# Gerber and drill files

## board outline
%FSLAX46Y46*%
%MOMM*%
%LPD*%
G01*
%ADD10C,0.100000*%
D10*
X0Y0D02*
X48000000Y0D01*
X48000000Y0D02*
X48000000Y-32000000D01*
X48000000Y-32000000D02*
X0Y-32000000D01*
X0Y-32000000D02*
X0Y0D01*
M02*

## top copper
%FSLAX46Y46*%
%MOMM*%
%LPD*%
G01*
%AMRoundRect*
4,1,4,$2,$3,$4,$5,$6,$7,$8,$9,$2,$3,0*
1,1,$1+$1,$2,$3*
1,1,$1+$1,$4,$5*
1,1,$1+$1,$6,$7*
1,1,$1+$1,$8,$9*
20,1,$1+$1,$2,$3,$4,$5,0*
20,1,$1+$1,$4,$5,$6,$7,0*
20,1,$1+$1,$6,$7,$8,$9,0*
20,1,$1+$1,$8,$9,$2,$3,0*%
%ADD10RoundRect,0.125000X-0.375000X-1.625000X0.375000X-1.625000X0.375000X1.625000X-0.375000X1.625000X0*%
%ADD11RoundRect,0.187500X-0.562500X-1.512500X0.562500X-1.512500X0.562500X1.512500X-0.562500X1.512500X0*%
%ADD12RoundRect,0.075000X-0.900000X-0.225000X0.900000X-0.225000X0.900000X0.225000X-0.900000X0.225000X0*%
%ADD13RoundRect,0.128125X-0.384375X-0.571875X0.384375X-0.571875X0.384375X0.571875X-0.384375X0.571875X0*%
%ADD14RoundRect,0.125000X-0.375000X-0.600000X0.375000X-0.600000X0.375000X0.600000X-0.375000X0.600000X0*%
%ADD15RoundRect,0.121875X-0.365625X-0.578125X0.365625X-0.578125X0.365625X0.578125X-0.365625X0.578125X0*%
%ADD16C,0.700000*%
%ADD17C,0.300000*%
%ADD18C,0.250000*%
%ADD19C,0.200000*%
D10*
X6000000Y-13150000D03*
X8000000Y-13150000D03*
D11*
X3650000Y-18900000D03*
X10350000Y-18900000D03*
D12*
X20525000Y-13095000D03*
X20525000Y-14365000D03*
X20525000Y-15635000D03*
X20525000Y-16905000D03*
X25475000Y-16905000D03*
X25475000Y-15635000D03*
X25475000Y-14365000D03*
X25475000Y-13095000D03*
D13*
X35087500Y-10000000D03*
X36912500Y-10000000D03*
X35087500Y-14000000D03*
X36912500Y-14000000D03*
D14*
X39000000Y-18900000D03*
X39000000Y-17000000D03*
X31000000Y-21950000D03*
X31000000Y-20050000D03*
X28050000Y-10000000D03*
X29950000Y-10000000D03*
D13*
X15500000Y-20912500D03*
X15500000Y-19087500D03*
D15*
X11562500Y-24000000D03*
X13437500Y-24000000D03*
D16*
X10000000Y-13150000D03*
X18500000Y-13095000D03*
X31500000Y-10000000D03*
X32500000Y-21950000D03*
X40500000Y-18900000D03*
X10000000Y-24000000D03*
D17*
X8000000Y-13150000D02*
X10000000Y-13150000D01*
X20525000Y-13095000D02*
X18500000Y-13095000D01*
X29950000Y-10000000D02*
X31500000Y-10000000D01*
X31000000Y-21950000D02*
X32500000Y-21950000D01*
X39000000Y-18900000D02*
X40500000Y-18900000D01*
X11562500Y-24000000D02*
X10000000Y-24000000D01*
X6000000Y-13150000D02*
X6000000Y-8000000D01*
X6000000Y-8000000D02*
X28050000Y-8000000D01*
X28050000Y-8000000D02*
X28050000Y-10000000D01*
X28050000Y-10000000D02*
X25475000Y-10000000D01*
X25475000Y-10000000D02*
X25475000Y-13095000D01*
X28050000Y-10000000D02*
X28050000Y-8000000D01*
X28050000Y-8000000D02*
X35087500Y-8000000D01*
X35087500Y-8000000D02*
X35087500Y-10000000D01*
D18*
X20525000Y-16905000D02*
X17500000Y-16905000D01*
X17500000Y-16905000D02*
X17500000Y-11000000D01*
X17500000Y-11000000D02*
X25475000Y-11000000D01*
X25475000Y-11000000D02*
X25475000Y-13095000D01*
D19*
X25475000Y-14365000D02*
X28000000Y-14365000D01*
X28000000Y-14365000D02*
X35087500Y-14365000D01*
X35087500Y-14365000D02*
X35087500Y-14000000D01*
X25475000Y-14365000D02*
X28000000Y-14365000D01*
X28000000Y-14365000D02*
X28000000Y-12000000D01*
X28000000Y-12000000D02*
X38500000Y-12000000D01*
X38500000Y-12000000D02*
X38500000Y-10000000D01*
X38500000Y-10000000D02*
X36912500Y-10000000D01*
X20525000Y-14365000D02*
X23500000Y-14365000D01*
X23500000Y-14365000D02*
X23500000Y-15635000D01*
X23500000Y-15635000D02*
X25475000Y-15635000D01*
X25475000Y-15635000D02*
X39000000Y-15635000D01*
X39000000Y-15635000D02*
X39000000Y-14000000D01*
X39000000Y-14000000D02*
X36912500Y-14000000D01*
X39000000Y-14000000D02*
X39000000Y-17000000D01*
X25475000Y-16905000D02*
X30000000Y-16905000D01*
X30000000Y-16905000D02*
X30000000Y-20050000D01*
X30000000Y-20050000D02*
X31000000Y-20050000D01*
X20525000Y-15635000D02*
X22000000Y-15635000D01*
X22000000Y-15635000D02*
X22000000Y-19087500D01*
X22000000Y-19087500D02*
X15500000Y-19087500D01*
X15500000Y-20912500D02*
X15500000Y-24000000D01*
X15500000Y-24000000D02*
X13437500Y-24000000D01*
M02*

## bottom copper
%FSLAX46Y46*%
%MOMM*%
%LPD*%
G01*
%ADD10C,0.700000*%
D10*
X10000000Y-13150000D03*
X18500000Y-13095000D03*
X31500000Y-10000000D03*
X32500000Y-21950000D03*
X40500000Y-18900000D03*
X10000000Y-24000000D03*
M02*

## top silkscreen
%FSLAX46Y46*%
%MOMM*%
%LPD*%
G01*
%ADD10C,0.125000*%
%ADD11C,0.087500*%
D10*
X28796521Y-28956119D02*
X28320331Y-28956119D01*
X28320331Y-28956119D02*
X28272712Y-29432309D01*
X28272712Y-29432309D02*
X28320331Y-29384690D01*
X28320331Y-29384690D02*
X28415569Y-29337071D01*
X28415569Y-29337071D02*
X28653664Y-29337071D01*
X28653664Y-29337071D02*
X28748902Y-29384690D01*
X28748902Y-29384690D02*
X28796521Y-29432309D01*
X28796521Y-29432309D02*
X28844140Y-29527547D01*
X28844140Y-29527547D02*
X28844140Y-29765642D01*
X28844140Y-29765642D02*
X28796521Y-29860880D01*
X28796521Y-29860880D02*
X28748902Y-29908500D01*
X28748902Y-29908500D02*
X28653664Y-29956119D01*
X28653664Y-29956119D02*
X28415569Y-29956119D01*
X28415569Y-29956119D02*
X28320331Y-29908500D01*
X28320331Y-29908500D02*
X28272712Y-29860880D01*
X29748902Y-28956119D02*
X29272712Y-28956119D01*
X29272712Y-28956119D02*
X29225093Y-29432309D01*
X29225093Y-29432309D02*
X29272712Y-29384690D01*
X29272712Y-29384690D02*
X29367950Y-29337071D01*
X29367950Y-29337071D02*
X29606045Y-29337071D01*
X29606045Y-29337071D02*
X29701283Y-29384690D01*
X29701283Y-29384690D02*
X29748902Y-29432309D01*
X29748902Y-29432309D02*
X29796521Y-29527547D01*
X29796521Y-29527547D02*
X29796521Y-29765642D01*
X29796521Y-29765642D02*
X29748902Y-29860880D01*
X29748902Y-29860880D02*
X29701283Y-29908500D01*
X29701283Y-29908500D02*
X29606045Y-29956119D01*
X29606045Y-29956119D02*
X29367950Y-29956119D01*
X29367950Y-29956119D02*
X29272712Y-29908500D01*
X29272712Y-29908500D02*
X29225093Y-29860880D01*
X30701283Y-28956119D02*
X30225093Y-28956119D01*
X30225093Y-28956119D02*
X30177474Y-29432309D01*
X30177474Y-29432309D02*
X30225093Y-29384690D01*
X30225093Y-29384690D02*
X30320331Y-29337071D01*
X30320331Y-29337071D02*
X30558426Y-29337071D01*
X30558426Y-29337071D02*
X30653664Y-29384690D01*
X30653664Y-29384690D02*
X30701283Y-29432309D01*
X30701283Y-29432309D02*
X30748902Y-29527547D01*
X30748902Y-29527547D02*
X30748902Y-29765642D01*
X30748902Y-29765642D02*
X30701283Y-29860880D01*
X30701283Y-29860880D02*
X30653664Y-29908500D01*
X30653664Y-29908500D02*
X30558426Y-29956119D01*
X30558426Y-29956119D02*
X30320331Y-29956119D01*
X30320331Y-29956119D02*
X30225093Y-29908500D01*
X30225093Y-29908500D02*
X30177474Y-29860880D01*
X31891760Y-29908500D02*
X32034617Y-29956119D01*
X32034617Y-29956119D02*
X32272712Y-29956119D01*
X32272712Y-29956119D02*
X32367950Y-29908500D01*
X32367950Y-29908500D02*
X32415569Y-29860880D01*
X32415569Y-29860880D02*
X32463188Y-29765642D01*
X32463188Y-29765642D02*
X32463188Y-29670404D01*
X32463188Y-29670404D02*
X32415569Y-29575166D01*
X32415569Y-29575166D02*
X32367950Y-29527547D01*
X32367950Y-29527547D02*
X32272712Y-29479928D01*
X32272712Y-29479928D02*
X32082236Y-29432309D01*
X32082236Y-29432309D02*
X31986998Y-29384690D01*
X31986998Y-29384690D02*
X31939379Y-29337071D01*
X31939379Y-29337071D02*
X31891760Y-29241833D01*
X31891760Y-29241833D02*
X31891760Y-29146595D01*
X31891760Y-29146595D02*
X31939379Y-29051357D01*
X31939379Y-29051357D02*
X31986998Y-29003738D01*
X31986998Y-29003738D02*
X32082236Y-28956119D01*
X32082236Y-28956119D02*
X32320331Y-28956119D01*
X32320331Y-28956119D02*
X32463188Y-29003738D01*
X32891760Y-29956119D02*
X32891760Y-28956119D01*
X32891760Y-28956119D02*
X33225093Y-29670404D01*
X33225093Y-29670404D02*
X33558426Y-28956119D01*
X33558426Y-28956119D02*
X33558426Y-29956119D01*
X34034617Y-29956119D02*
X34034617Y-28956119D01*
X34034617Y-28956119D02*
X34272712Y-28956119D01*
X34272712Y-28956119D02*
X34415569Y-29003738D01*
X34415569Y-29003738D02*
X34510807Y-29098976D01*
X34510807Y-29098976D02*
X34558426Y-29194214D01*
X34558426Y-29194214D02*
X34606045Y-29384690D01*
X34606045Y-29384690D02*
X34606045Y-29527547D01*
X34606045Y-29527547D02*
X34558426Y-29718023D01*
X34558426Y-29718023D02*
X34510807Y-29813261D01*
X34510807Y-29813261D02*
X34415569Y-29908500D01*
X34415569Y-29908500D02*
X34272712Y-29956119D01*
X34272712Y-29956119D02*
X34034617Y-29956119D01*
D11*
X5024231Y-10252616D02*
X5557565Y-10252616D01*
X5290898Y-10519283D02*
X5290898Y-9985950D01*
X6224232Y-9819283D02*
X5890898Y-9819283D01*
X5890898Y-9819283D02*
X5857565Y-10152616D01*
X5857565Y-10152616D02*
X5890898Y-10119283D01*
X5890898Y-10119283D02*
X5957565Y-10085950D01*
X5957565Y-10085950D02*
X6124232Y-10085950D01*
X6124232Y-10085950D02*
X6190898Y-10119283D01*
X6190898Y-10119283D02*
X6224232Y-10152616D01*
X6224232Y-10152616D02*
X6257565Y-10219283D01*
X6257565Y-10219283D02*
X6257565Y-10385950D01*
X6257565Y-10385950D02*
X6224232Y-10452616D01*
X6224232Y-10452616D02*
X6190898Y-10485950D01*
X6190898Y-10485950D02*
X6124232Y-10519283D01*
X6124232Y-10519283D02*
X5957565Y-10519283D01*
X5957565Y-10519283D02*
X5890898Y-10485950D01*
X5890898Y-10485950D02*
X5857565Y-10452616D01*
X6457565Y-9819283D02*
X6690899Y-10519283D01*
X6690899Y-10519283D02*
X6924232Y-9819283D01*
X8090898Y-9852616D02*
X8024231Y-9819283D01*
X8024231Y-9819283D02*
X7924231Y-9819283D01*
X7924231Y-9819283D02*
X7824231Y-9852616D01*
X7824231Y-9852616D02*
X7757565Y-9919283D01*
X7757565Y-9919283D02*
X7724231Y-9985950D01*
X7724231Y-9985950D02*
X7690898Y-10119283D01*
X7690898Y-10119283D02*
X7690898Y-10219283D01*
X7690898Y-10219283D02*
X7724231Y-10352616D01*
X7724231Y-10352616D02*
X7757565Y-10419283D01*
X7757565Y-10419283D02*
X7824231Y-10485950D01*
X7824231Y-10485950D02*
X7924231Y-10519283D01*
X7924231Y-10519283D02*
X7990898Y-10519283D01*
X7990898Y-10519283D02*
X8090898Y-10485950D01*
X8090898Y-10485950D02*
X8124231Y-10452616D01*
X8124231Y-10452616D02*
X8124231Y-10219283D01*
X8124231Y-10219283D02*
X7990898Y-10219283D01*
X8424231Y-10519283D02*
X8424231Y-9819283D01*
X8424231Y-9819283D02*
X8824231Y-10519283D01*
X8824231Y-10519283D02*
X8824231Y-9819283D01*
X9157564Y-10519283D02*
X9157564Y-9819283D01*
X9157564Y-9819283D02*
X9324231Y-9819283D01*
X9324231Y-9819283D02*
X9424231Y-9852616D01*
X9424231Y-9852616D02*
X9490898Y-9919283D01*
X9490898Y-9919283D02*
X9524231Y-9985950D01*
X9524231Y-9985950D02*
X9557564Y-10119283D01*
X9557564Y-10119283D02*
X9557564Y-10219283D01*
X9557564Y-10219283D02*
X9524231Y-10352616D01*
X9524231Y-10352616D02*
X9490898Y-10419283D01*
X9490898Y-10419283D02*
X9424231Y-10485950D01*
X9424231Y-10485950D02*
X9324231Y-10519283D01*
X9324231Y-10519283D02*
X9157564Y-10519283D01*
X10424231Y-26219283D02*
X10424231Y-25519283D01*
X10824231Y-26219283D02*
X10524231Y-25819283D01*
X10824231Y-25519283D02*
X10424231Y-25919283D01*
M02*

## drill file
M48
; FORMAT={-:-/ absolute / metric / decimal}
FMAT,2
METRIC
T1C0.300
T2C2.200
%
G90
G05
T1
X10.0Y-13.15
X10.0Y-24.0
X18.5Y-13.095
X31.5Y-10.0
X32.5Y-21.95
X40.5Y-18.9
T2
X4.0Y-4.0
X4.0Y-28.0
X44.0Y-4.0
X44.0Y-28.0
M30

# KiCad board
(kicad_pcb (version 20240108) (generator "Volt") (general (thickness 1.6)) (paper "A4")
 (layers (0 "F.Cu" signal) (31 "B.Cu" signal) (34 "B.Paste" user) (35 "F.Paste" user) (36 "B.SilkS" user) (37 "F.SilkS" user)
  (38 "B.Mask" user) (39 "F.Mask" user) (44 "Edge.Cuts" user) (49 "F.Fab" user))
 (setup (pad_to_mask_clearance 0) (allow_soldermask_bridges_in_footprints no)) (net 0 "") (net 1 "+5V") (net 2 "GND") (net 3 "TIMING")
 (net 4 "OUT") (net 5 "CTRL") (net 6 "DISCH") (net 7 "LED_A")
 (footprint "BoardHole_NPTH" (layer "F.Cu") (at 4 4)
  (pad "" np_thru_hole circle (at 0 0) (size 2.2 2.2) (drill 2.2) (layers "*.Cu" "*.Mask")))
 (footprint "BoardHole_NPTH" (layer "F.Cu") (at 44 4)
  (pad "" np_thru_hole circle (at 0 0) (size 2.2 2.2) (drill 2.2) (layers "*.Cu" "*.Mask")))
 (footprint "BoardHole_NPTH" (layer "F.Cu") (at 4 28)
  (pad "" np_thru_hole circle (at 0 0) (size 2.2 2.2) (drill 2.2) (layers "*.Cu" "*.Mask")))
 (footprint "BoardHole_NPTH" (layer "F.Cu") (at 44 28)
  (pad "" np_thru_hole circle (at 0 0) (size 2.2 2.2) (drill 2.2) (layers "*.Cu" "*.Mask")))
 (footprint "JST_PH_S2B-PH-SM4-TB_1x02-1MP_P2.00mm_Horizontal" (layer "F.Cu") (at 7 16)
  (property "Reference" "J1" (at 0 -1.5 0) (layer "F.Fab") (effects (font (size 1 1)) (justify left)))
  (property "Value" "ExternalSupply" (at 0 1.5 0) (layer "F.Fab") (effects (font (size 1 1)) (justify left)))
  (pad "1" smd roundrect (at -1 -2.85) (size 1 3.5) (layers "F.Cu" "F.Paste" "F.Mask") (roundrect_rratio 0.125) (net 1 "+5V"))
  (pad "2" smd roundrect (at 1 -2.85) (size 1 3.5) (layers "F.Cu" "F.Paste" "F.Mask") (roundrect_rratio 0.125) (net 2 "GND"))
  (pad "MP1" smd roundrect (at -3.35 2.9) (size 1.5 3.4) (layers "F.Cu" "F.Paste" "F.Mask") (roundrect_rratio 0.125))
  (pad "MP2" smd roundrect (at 3.35 2.9) (size 1.5 3.4) (layers "F.Cu" "F.Paste" "F.Mask") (roundrect_rratio 0.125)))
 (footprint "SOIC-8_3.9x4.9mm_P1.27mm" (layer "F.Cu") (at 23 15)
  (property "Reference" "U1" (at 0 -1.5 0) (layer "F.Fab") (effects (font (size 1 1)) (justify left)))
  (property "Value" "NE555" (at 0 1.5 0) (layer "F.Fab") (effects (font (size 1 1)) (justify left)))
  (pad "1" smd roundrect (at -2.475 -1.905) (size 1.95 0.6) (layers "F.Cu" "F.Paste" "F.Mask") (roundrect_rratio 0.125) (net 2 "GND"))
  (pad "2" smd roundrect (at -2.475 -0.635) (size 1.95 0.6) (layers "F.Cu" "F.Paste" "F.Mask") (roundrect_rratio 0.125) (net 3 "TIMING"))
  (pad "3" smd roundrect (at -2.475 0.635) (size 1.95 0.6) (layers "F.Cu" "F.Paste" "F.Mask") (roundrect_rratio 0.125) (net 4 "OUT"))
  (pad "4" smd roundrect (at -2.475 1.905) (size 1.95 0.6) (layers "F.Cu" "F.Paste" "F.Mask") (roundrect_rratio 0.125) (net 1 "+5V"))
  (pad "5" smd roundrect (at 2.475 1.905) (size 1.95 0.6) (layers "F.Cu" "F.Paste" "F.Mask") (roundrect_rratio 0.125) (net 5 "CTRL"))
  (pad "6" smd roundrect (at 2.475 0.635) (size 1.95 0.6) (layers "F.Cu" "F.Paste" "F.Mask") (roundrect_rratio 0.125) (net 3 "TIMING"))
  (pad "7" smd roundrect (at 2.475 -0.635) (size 1.95 0.6) (layers "F.Cu" "F.Paste" "F.Mask") (roundrect_rratio 0.125) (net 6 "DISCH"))
  (pad "8" smd roundrect (at 2.475 -1.905) (size 1.95 0.6) (layers "F.Cu" "F.Paste" "F.Mask") (roundrect_rratio 0.125) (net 1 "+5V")))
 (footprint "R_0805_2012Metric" (layer "F.Cu") (at 36 10)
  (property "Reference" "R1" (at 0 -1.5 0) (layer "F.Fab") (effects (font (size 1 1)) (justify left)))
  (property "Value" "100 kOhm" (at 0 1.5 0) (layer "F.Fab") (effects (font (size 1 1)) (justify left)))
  (pad "1" smd roundrect (at -0.9125 0) (size 1.025 1.4) (layers "F.Cu" "F.Paste" "F.Mask") (roundrect_rratio 0.125) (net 1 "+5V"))
  (pad "2" smd roundrect (at 0.9125 0) (size 1.025 1.4) (layers "F.Cu" "F.Paste" "F.Mask") (roundrect_rratio 0.125) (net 6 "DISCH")))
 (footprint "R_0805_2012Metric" (layer "F.Cu") (at 36 14)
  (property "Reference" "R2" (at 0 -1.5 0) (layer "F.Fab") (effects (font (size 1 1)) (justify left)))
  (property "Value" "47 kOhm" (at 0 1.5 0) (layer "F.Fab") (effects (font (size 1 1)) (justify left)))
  (pad "1" smd roundrect (at -0.9125 0) (size 1.025 1.4) (layers "F.Cu" "F.Paste" "F.Mask") (roundrect_rratio 0.125) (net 6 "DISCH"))
  (pad "2" smd roundrect (at 0.9125 0) (size 1.025 1.4) (layers "F.Cu" "F.Paste" "F.Mask") (roundrect_rratio 0.125) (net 3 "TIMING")))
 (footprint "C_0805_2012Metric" (layer "F.Cu") (at 39 17.95 90)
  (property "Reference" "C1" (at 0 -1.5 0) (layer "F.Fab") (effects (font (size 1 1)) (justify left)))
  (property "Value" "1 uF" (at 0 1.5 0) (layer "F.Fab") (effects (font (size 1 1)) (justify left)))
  (pad "1" smd roundrect (at -0.95 0) (size 1 1.45) (layers "F.Cu" "F.Paste" "F.Mask") (roundrect_rratio 0.125) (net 3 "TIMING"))
  (pad "2" smd roundrect (at 0.95 0) (size 1 1.45) (layers "F.Cu" "F.Paste" "F.Mask") (roundrect_rratio 0.125) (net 2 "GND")))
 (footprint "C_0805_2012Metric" (layer "F.Cu") (at 31 21 90)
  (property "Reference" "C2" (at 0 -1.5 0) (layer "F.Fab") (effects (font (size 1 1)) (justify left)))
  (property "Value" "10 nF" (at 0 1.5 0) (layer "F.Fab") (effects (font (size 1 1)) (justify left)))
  (pad "1" smd roundrect (at -0.95 0) (size 1 1.45) (layers "F.Cu" "F.Paste" "F.Mask") (roundrect_rratio 0.125) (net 5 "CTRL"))
  (pad "2" smd roundrect (at 0.95 0) (size 1 1.45) (layers "F.Cu" "F.Paste" "F.Mask") (roundrect_rratio 0.125) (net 2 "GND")))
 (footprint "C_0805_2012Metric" (layer "F.Cu") (at 29 10)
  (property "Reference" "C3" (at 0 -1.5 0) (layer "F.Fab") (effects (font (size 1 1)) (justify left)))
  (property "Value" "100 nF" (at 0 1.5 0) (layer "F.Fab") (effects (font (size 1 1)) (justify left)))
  (pad "1" smd roundrect (at -0.95 0) (size 1 1.45) (layers "F.Cu" "F.Paste" "F.Mask") (roundrect_rratio 0.125) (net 1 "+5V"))
  (pad "2" smd roundrect (at 0.95 0) (size 1 1.45) (layers "F.Cu" "F.Paste" "F.Mask") (roundrect_rratio 0.125) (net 2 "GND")))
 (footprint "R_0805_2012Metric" (layer "F.Cu") (at 15.5 20 90)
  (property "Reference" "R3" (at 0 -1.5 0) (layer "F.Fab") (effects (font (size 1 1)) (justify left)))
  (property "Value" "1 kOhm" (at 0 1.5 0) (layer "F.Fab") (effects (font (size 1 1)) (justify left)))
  (pad "1" smd roundrect (at -0.9125 0) (size 1.025 1.4) (layers "F.Cu" "F.Paste" "F.Mask") (roundrect_rratio 0.125) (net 4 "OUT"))
  (pad "2" smd roundrect (at 0.9125 0) (size 1.025 1.4) (layers "F.Cu" "F.Paste" "F.Mask") (roundrect_rratio 0.125) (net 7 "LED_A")))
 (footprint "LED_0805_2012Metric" (layer "F.Cu") (at 12.5 24)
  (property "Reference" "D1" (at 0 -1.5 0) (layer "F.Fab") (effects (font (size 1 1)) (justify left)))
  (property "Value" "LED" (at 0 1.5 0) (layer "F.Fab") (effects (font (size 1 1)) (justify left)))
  (pad "1" smd roundrect (at -0.9375 0) (size 0.975 1.4) (layers "F.Cu" "F.Paste" "F.Mask") (roundrect_rratio 0.125) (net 2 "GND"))
  (pad "2" smd roundrect (at 0.9375 0) (size 0.975 1.4) (layers "F.Cu" "F.Paste" "F.Mask") (roundrect_rratio 0.125) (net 7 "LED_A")))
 (segment (start 8 13.15) (end 10 13.15) (width 0.3) (layer "F.Cu") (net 2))
 (segment (start 20.525 13.095) (end 18.5 13.095) (width 0.3) (layer "F.Cu") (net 2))
 (segment (start 29.95 10) (end 31.5 10) (width 0.3) (layer "F.Cu") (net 2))
 (segment (start 31 21.95) (end 32.5 21.95) (width 0.3) (layer "F.Cu") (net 2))
 (segment (start 39 18.9) (end 40.5 18.9) (width 0.3) (layer "F.Cu") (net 2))
 (segment (start 11.5625 24) (end 10 24) (width 0.3) (layer "F.Cu") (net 2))
 (segment (start 6 13.15) (end 6 8) (width 0.3) (layer "F.Cu") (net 1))
 (segment (start 6 8) (end 28.05 8) (width 0.3) (layer "F.Cu") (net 1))
 (segment (start 28.05 8) (end 28.05 10) (width 0.3) (layer "F.Cu") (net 1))
 (segment (start 28.05 10) (end 25.475 10) (width 0.3) (layer "F.Cu") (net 1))
 (segment (start 25.475 10) (end 25.475 13.095) (width 0.3) (layer "F.Cu") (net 1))
 (segment (start 28.05 10) (end 28.05 8) (width 0.3) (layer "F.Cu") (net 1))
 (segment (start 28.05 8) (end 35.0875 8) (width 0.3) (layer "F.Cu") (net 1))
 (segment (start 35.0875 8) (end 35.0875 10) (width 0.3) (layer "F.Cu") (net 1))
 (segment (start 20.525 16.905) (end 17.5 16.905) (width 0.25) (layer "F.Cu") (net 1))
 (segment (start 17.5 16.905) (end 17.5 11) (width 0.25) (layer "F.Cu") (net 1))
 (segment (start 17.5 11) (end 25.475 11) (width 0.25) (layer "F.Cu") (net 1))
 (segment (start 25.475 11) (end 25.475 13.095) (width 0.25) (layer "F.Cu") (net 1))
 (segment (start 25.475 14.365) (end 28 14.365) (width 0.2) (layer "F.Cu") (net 6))
 (segment (start 28 14.365) (end 35.0875 14.365) (width 0.2) (layer "F.Cu") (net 6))
 (segment (start 35.0875 14.365) (end 35.0875 14) (width 0.2) (layer "F.Cu") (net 6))
 (segment (start 25.475 14.365) (end 28 14.365) (width 0.2) (layer "F.Cu") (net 6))
 (segment (start 28 14.365) (end 28 12) (width 0.2) (layer "F.Cu") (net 6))
 (segment (start 28 12) (end 38.5 12) (width 0.2) (layer "F.Cu") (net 6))
 (segment (start 38.5 12) (end 38.5 10) (width 0.2) (layer "F.Cu") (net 6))
 (segment (start 38.5 10) (end 36.9125 10) (width 0.2) (layer "F.Cu") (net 6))
 (segment (start 20.525 14.365) (end 23.5 14.365) (width 0.2) (layer "F.Cu") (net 3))
 (segment (start 23.5 14.365) (end 23.5 15.635) (width 0.2) (layer "F.Cu") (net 3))
 (segment (start 23.5 15.635) (end 25.475 15.635) (width 0.2) (layer "F.Cu") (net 3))
 (segment (start 25.475 15.635) (end 39 15.635) (width 0.2) (layer "F.Cu") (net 3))
 (segment (start 39 15.635) (end 39 14) (width 0.2) (layer "F.Cu") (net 3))
 (segment (start 39 14) (end 36.9125 14) (width 0.2) (layer "F.Cu") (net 3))
 (segment (start 39 14) (end 39 17) (width 0.2) (layer "F.Cu") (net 3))
 (segment (start 25.475 16.905) (end 30 16.905) (width 0.2) (layer "F.Cu") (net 5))
 (segment (start 30 16.905) (end 30 20.05) (width 0.2) (layer "F.Cu") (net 5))
 (segment (start 30 20.05) (end 31 20.05) (width 0.2) (layer "F.Cu") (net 5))
 (segment (start 20.525 15.635) (end 22 15.635) (width 0.2) (layer "F.Cu") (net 4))
 (segment (start 22 15.635) (end 22 19.0875) (width 0.2) (layer "F.Cu") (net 4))
 (segment (start 22 19.0875) (end 15.5 19.0875) (width 0.2) (layer "F.Cu") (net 4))
 (segment (start 15.5 20.9125) (end 15.5 24) (width 0.2) (layer "F.Cu") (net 7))
 (segment (start 15.5 24) (end 13.4375 24) (width 0.2) (layer "F.Cu") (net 7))
 (via (at 10 13.15) (size 0.7) (drill 0.3) (layers "F.Cu" "B.Cu") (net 2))
 (via (at 18.5 13.095) (size 0.7) (drill 0.3) (layers "F.Cu" "B.Cu") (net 2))
 (via (at 31.5 10) (size 0.7) (drill 0.3) (layers "F.Cu" "B.Cu") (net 2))
 (via (at 32.5 21.95) (size 0.7) (drill 0.3) (layers "F.Cu" "B.Cu") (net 2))
 (via (at 40.5 18.9) (size 0.7) (drill 0.3) (layers "F.Cu" "B.Cu") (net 2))
 (via (at 10 24) (size 0.7) (drill 0.3) (layers "F.Cu" "B.Cu") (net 2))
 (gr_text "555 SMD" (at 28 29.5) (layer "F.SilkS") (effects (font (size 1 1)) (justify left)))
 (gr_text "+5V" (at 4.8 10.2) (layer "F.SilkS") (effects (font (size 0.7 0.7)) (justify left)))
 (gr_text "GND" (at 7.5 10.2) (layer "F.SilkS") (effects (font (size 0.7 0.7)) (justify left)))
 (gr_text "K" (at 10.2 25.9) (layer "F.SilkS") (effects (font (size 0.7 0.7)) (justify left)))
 (gr_line (start 0 0) (end 48 0) (stroke (width 0.1) (type default)) (layer "Edge.Cuts"))
 (gr_line (start 48 0) (end 48 32) (stroke (width 0.1) (type default)) (layer "Edge.Cuts"))
 (gr_line (start 48 32) (end 0 32) (stroke (width 0.1) (type default)) (layer "Edge.Cuts"))
 (gr_line (start 0 32) (end 0 0) (stroke (width 0.1) (type default)) (layer "Edge.Cuts")))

